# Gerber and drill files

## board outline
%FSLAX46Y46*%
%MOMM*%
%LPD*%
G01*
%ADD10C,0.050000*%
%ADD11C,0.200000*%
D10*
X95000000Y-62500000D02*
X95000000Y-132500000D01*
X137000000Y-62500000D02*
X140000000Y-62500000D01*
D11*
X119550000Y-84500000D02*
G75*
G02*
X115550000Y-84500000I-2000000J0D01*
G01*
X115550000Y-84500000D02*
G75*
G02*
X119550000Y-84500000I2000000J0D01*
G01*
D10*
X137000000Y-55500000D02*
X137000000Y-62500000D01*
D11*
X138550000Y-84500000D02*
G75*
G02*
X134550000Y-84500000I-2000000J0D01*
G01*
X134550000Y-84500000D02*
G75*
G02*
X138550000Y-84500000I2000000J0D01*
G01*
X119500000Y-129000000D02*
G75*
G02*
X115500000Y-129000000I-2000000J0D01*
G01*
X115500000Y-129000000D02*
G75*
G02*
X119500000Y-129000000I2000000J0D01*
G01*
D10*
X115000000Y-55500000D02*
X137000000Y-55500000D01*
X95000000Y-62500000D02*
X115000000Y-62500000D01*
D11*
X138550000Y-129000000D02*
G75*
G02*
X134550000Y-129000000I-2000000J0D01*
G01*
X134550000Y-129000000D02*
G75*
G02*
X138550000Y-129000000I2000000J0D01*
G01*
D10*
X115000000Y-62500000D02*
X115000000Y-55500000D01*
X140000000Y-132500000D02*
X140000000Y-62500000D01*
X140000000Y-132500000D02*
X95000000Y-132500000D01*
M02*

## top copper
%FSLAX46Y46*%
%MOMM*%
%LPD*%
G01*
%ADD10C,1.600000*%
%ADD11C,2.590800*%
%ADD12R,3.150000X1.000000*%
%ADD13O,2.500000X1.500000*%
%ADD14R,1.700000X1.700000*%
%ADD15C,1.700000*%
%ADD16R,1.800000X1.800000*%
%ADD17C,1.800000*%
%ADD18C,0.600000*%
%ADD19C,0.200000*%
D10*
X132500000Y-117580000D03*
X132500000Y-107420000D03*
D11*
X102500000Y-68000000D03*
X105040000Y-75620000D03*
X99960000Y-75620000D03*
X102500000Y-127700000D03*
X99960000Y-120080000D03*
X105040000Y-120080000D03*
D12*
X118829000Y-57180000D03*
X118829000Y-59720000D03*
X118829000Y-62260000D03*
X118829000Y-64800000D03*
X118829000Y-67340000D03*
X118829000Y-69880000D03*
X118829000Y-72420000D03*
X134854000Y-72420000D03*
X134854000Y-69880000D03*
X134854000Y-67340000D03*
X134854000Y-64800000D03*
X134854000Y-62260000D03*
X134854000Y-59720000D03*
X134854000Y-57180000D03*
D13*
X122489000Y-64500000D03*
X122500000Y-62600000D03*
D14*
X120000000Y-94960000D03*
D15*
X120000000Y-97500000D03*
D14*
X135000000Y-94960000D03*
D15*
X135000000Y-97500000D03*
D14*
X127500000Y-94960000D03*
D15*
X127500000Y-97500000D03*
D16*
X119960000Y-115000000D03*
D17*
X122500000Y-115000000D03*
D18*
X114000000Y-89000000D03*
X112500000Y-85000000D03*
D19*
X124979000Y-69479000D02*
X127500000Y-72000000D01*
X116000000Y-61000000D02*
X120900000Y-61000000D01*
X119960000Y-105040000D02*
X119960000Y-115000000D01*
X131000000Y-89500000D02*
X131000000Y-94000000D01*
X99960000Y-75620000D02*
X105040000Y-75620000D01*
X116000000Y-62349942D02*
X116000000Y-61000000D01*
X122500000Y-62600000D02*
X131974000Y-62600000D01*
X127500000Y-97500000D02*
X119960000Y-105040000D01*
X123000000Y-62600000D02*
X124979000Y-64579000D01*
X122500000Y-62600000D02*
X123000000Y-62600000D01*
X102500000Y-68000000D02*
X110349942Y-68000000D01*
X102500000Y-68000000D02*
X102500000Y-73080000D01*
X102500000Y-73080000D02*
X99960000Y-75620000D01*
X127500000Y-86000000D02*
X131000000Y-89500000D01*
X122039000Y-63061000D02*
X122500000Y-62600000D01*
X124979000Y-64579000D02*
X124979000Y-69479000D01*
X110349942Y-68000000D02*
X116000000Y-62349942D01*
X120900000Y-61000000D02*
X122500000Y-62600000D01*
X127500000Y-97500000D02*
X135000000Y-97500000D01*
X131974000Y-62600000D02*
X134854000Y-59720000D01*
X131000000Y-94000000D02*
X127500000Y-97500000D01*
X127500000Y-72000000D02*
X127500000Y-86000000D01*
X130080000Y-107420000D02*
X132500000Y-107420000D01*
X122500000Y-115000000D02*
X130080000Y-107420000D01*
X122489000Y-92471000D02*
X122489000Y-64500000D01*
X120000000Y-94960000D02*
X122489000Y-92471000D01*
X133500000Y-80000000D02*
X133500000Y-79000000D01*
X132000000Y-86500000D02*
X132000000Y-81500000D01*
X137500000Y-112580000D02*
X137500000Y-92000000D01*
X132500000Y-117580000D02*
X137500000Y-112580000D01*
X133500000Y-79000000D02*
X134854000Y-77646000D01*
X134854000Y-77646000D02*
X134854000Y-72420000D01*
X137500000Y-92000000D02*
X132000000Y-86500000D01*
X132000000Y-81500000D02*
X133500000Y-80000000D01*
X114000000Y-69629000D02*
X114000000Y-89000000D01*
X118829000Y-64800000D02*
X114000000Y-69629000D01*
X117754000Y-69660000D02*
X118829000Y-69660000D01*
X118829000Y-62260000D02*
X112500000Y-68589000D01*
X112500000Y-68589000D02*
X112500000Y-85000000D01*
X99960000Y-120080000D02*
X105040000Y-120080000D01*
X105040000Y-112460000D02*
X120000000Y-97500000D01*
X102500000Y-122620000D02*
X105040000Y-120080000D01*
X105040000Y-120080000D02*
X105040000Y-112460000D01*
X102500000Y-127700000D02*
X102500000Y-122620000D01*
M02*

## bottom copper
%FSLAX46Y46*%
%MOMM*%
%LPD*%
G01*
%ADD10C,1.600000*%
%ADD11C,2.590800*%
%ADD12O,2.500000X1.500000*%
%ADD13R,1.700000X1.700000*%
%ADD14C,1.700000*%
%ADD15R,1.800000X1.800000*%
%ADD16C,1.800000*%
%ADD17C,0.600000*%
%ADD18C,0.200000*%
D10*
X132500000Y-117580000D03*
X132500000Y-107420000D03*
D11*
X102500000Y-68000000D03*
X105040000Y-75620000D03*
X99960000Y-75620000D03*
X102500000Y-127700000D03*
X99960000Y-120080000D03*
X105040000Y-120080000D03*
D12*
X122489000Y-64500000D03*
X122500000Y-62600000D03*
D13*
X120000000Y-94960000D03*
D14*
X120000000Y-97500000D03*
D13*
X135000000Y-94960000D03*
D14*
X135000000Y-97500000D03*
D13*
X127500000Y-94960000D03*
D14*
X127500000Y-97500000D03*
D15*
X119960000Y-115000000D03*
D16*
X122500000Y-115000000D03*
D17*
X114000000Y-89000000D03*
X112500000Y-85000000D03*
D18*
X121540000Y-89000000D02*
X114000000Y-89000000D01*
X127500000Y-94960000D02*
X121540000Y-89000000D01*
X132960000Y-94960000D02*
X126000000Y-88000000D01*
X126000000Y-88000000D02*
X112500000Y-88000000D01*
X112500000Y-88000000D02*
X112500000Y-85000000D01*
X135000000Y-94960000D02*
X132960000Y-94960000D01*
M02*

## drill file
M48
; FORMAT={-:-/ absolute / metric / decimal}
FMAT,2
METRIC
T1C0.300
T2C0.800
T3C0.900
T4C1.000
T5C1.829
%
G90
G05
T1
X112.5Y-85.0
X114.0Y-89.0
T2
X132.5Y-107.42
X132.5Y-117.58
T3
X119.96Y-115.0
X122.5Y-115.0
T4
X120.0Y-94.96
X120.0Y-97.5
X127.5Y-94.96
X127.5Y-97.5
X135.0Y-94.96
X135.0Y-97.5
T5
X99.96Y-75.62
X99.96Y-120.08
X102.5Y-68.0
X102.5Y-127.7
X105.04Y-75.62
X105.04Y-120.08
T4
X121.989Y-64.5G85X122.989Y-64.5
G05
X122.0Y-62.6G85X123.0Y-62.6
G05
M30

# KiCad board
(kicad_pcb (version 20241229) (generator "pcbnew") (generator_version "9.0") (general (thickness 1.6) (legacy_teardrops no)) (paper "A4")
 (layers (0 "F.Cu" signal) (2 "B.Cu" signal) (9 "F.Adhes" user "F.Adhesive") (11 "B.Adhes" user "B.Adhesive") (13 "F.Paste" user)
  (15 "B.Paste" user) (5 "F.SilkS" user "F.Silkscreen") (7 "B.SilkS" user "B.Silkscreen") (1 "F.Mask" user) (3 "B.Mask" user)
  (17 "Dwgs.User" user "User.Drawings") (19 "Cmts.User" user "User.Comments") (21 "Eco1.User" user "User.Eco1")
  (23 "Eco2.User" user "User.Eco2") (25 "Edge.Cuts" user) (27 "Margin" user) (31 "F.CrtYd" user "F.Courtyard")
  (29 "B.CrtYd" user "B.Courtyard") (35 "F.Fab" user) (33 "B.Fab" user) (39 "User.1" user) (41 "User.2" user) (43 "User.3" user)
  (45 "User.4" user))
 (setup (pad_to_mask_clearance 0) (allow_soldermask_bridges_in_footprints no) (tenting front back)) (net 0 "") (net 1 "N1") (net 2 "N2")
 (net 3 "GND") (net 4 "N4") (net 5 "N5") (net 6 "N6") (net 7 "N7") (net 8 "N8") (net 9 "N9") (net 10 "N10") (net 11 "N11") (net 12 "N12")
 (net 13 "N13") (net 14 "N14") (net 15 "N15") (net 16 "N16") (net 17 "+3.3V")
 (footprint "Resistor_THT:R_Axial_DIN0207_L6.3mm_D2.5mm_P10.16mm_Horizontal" (layer "F.Cu") (at 132.5 117.58 90)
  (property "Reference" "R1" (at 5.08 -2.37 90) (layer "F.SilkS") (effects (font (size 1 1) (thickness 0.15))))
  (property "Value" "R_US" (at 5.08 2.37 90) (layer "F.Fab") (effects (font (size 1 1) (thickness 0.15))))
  (pad "1" thru_hole circle (at 0 0 90) (size 1.6 1.6) (drill 0.8) (layers "*.Cu" "*.Mask") (remove_unused_layers no) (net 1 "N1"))
  (pad "2" thru_hole circle (at 10.16 0 90) (size 1.6 1.6) (drill 0.8) (layers "*.Cu" "*.Mask") (remove_unused_layers no) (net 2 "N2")))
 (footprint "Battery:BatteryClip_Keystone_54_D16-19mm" (layer "F.Cu") (at 102.5 68 -90)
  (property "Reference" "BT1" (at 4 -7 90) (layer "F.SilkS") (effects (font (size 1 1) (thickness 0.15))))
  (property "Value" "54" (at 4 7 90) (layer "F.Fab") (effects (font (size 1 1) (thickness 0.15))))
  (pad "1" thru_hole circle (at 0 0 90) (size 2.5908 2.5908) (drill 1.8288) (layers "*.Cu" "*.Mask") (remove_unused_layers no) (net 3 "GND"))
  (pad "1" thru_hole circle (at 7.62 -2.54 90) (size 2.5908 2.5908) (drill 1.8288) (layers "*.Cu" "*.Mask") (remove_unused_layers no)
   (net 3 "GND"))
  (pad "1" thru_hole circle (at 7.62 2.54 90) (size 2.5908 2.5908) (drill 1.8288) (layers "*.Cu" "*.Mask") (remove_unused_layers no)
   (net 3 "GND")))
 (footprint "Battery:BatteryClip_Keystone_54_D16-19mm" (layer "F.Cu") (at 102.5 127.7 90)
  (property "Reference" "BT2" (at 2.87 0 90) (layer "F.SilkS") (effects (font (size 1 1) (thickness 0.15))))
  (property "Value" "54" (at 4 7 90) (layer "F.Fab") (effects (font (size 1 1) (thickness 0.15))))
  (pad "1" thru_hole circle (at 0 0 270) (size 2.5908 2.5908) (drill 1.8288) (layers "*.Cu" "*.Mask") (remove_unused_layers no) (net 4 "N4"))
  (pad "1" thru_hole circle (at 7.62 -2.54 270) (size 2.5908 2.5908) (drill 1.8288) (layers "*.Cu" "*.Mask") (remove_unused_layers no)
   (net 4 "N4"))
  (pad "1" thru_hole circle (at 7.62 2.54 270) (size 2.5908 2.5908) (drill 1.8288) (layers "*.Cu" "*.Mask") (remove_unused_layers no)
   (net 4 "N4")))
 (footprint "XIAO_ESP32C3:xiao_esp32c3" (layer "F.Cu") (at 127.429 66.6)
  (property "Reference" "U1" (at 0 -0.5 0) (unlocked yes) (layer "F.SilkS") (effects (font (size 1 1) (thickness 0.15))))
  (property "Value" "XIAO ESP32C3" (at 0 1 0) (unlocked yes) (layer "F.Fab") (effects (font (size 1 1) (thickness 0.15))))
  (pad "1" smd rect (at -8.6 -9.42) (size 3.15 1) (layers "F.Cu" "F.Mask" "F.Paste") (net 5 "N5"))
  (pad "2" smd rect (at -8.6 -6.88) (size 3.15 1) (layers "F.Cu" "F.Mask" "F.Paste") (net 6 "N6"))
  (pad "3" smd rect (at -8.6 -4.34) (size 3.15 1) (layers "F.Cu" "F.Mask" "F.Paste") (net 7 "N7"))
  (pad "4" smd rect (at -8.6 -1.8) (size 3.15 1) (layers "F.Cu" "F.Mask" "F.Paste") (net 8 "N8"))
  (pad "5" smd rect (at -8.6 0.74) (size 3.15 1) (layers "F.Cu" "F.Mask" "F.Paste") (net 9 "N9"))
  (pad "6" smd rect (at -8.6 3.28) (size 3.15 1) (layers "F.Cu" "F.Mask" "F.Paste") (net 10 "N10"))
  (pad "7" smd rect (at -8.6 5.82) (size 3.15 1) (layers "F.Cu" "F.Mask" "F.Paste") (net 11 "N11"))
  (pad "8" smd rect (at 7.425 5.82) (size 3.15 1) (layers "F.Cu" "F.Mask" "F.Paste") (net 1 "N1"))
  (pad "9" smd rect (at 7.425 3.28) (size 3.15 1) (layers "F.Cu" "F.Mask" "F.Paste") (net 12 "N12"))
  (pad "10" smd rect (at 7.425 0.74) (size 3.15 1) (layers "F.Cu" "F.Mask" "F.Paste") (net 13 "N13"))
  (pad "11" smd rect (at 7.425 -1.8) (size 3.15 1) (layers "F.Cu" "F.Mask" "F.Paste") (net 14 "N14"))
  (pad "12" smd rect (at 7.425 -4.34) (size 3.15 1) (layers "F.Cu" "F.Mask" "F.Paste") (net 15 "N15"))
  (pad "13" smd rect (at 7.425 -6.88) (size 3.15 1) (layers "F.Cu" "F.Mask" "F.Paste") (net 3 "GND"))
  (pad "14" smd rect (at 7.425 -9.42) (size 3.15 1) (layers "F.Cu" "F.Mask" "F.Paste") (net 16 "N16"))
  (pad "B+" thru_hole oval (at -4.94 -2.1) (size 2.5 1.5) (drill oval 2 1) (layers "*.Cu" "*.Mask") (remove_unused_layers no)
   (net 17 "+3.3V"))
  (pad "B-" thru_hole oval (at -4.929 -4) (size 2.5 1.5) (drill oval 2 1) (layers "*.Cu" "*.Mask") (remove_unused_layers no) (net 3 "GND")))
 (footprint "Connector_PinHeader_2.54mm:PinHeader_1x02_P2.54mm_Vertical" (layer "F.Cu") (at 120 94.96)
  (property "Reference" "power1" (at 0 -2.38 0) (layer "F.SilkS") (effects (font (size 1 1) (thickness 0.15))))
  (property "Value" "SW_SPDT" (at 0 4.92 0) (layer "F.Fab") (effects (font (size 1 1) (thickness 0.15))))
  (pad "1" thru_hole rect (at 0 0) (size 1.7 1.7) (drill 1) (layers "*.Cu" "*.Mask") (remove_unused_layers no) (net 17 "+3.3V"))
  (pad "2" thru_hole circle (at 0 2.54) (size 1.7 1.7) (drill 1) (layers "*.Cu" "*.Mask") (remove_unused_layers no) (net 4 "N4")))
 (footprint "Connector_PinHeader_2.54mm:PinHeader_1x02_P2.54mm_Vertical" (layer "F.Cu") (at 135 94.96)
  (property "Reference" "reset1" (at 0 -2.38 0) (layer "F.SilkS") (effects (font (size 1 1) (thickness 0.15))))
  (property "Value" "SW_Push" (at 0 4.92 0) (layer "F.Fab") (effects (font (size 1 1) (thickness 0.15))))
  (pad "1" thru_hole rect (at 0 0) (size 1.7 1.7) (drill 1) (layers "*.Cu" "*.Mask") (remove_unused_layers no) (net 7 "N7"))
  (pad "2" thru_hole circle (at 0 2.54) (size 1.7 1.7) (drill 1) (layers "*.Cu" "*.Mask") (remove_unused_layers no) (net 3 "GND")))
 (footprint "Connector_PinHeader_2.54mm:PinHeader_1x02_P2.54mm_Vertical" (layer "F.Cu") (at 127.5 94.96)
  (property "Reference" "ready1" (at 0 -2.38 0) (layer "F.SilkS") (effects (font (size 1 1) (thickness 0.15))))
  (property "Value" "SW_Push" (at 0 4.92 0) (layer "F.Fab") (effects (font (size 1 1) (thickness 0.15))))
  (pad "1" thru_hole rect (at 0 0) (size 1.7 1.7) (drill 1) (layers "*.Cu" "*.Mask") (remove_unused_layers no) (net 8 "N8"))
  (pad "2" thru_hole circle (at 0 2.54) (size 1.7 1.7) (drill 1) (layers "*.Cu" "*.Mask") (remove_unused_layers no) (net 3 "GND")))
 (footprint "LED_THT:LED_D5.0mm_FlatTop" (layer "F.Cu") (at 119.96 115)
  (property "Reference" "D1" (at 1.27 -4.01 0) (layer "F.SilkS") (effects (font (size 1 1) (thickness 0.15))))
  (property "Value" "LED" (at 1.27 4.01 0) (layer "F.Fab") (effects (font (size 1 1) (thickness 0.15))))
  (pad "1" thru_hole rect (at 0 0) (size 1.8 1.8) (drill 0.9) (layers "*.Cu" "*.Mask") (remove_unused_layers no) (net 3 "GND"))
  (pad "2" thru_hole circle (at 2.54 0) (size 1.8 1.8) (drill 0.9) (layers "*.Cu" "*.Mask") (remove_unused_layers no) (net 2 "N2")))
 (gr_line (start 95 62.5) (end 95 132.5) (stroke (width 0.05) (type default)) (layer "Edge.Cuts"))
 (gr_line (start 137 62.5) (end 140 62.5) (stroke (width 0.05) (type default)) (layer "Edge.Cuts"))
 (gr_circle (center 117.55 84.5) (end 119.55 84.5) (stroke (width 0.2) (type solid)) (fill no) (layer "Edge.Cuts"))
 (gr_line (start 137 55.5) (end 137 62.5) (stroke (width 0.05) (type default)) (layer "Edge.Cuts"))
 (gr_circle (center 136.55 84.5) (end 138.55 84.5) (stroke (width 0.2) (type solid)) (fill no) (layer "Edge.Cuts"))
 (gr_circle (center 117.5 129) (end 119.5 129) (stroke (width 0.2) (type solid)) (fill no) (layer "Edge.Cuts"))
 (gr_line (start 115 55.5) (end 137 55.5) (stroke (width 0.05) (type default)) (layer "Edge.Cuts"))
 (gr_line (start 95 62.5) (end 115 62.5) (stroke (width 0.05) (type default)) (layer "Edge.Cuts"))
 (gr_circle (center 136.55 129) (end 138.55 129) (stroke (width 0.2) (type solid)) (fill no) (layer "Edge.Cuts"))
 (gr_line (start 115 62.5) (end 115 55.5) (stroke (width 0.05) (type default)) (layer "Edge.Cuts"))
 (gr_line (start 140 132.5) (end 140 62.5) (stroke (width 0.05) (type default)) (layer "Edge.Cuts"))
 (gr_line (start 140 132.5) (end 95 132.5) (stroke (width 0.05) (type default)) (layer "Edge.Cuts"))
 (segment (start 124.979 69.479) (end 127.5 72) (width 0.2) (layer "F.Cu") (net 3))
 (segment (start 116 61) (end 120.9 61) (width 0.2) (layer "F.Cu") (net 3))
 (segment (start 119.96 105.04) (end 119.96 115) (width 0.2) (layer "F.Cu") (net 3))
 (segment (start 131 89.5) (end 131 94) (width 0.2) (layer "F.Cu") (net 3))
 (segment (start 99.96 75.62) (end 105.04 75.62) (width 0.2) (layer "F.Cu") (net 3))
 (segment (start 116 62.349942) (end 116 61) (width 0.2) (layer "F.Cu") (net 3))
 (segment (start 122.5 62.6) (end 131.974 62.6) (width 0.2) (layer "F.Cu") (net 3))
 (segment (start 127.5 97.5) (end 119.96 105.04) (width 0.2) (layer "F.Cu") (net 3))
 (segment (start 123 62.6) (end 124.979 64.579) (width 0.2) (layer "F.Cu") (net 3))
 (segment (start 122.5 62.6) (end 123 62.6) (width 0.2) (layer "F.Cu") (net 3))
 (segment (start 102.5 68) (end 110.349942 68) (width 0.2) (layer "F.Cu") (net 3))
 (segment (start 102.5 68) (end 102.5 73.08) (width 0.2) (layer "F.Cu") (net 3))
 (segment (start 102.5 73.08) (end 99.96 75.62) (width 0.2) (layer "F.Cu") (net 3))
 (segment (start 127.5 86) (end 131 89.5) (width 0.2) (layer "F.Cu") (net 3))
 (segment (start 122.039 63.061) (end 122.5 62.6) (width 0.2) (layer "F.Cu") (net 3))
 (segment (start 124.979 64.579) (end 124.979 69.479) (width 0.2) (layer "F.Cu") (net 3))
 (segment (start 110.349942 68) (end 116 62.349942) (width 0.2) (layer "F.Cu") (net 3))
 (segment (start 120.9 61) (end 122.5 62.6) (width 0.2) (layer "F.Cu") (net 3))
 (segment (start 127.5 97.5) (end 135 97.5) (width 0.2) (layer "F.Cu") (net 3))
 (segment (start 131.974 62.6) (end 134.854 59.72) (width 0.2) (layer "F.Cu") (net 3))
 (segment (start 131 94) (end 127.5 97.5) (width 0.2) (layer "F.Cu") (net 3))
 (segment (start 127.5 72) (end 127.5 86) (width 0.2) (layer "F.Cu") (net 3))
 (segment (start 130.08 107.42) (end 132.5 107.42) (width 0.2) (layer "F.Cu") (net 2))
 (segment (start 122.5 115) (end 130.08 107.42) (width 0.2) (layer "F.Cu") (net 2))
 (segment (start 122.489 92.471) (end 122.489 64.5) (width 0.2) (layer "F.Cu") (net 17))
 (segment (start 120 94.96) (end 122.489 92.471) (width 0.2) (layer "F.Cu") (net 17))
 (segment (start 133.5 80) (end 133.5 79) (width 0.2) (layer "F.Cu") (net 1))
 (segment (start 132 86.5) (end 132 81.5) (width 0.2) (layer "F.Cu") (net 1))
 (segment (start 137.5 112.58) (end 137.5 92) (width 0.2) (layer "F.Cu") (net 1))
 (segment (start 132.5 117.58) (end 137.5 112.58) (width 0.2) (layer "F.Cu") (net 1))
 (segment (start 133.5 79) (end 134.854 77.646) (width 0.2) (layer "F.Cu") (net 1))
 (segment (start 134.854 77.646) (end 134.854 72.42) (width 0.2) (layer "F.Cu") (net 1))
 (segment (start 137.5 92) (end 132 86.5) (width 0.2) (layer "F.Cu") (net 1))
 (segment (start 132 81.5) (end 133.5 80) (width 0.2) (layer "F.Cu") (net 1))
 (segment (start 114 69.629) (end 114 89) (width 0.2) (layer "F.Cu") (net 8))
 (segment (start 118.829 64.8) (end 114 69.629) (width 0.2) (layer "F.Cu") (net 8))
 (via (at 114 89) (size 0.6) (drill 0.3) (layers "F.Cu" "B.Cu") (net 8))
 (segment (start 121.54 89) (end 114 89) (width 0.2) (layer "B.Cu") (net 8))
 (segment (start 127.5 94.96) (end 121.54 89) (width 0.2) (layer "B.Cu") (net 8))
 (segment (start 117.754 69.66) (end 118.829 69.66) (width 0.2) (layer "F.Cu") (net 10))
 (segment (start 118.829 62.26) (end 112.5 68.589) (width 0.2) (layer "F.Cu") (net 7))
 (segment (start 112.5 68.589) (end 112.5 85) (width 0.2) (layer "F.Cu") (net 7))
 (via (at 112.5 85) (size 0.6) (drill 0.3) (layers "F.Cu" "B.Cu") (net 7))
 (segment (start 132.96 94.96) (end 126 88) (width 0.2) (layer "B.Cu") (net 7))
 (segment (start 126 88) (end 112.5 88) (width 0.2) (layer "B.Cu") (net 7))
 (segment (start 112.5 88) (end 112.5 85) (width 0.2) (layer "B.Cu") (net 7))
 (segment (start 135 94.96) (end 132.96 94.96) (width 0.2) (layer "B.Cu") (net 7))
 (segment (start 99.96 120.08) (end 105.04 120.08) (width 0.2) (layer "F.Cu") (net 4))
 (segment (start 105.04 112.46) (end 120 97.5) (width 0.2) (layer "F.Cu") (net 4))
 (segment (start 102.5 122.62) (end 105.04 120.08) (width 0.2) (layer "F.Cu") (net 4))
 (segment (start 105.04 120.08) (end 105.04 112.46) (width 0.2) (layer "F.Cu") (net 4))
 (segment (start 102.5 127.7) (end 102.5 122.62) (width 0.2) (layer "F.Cu") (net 4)))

